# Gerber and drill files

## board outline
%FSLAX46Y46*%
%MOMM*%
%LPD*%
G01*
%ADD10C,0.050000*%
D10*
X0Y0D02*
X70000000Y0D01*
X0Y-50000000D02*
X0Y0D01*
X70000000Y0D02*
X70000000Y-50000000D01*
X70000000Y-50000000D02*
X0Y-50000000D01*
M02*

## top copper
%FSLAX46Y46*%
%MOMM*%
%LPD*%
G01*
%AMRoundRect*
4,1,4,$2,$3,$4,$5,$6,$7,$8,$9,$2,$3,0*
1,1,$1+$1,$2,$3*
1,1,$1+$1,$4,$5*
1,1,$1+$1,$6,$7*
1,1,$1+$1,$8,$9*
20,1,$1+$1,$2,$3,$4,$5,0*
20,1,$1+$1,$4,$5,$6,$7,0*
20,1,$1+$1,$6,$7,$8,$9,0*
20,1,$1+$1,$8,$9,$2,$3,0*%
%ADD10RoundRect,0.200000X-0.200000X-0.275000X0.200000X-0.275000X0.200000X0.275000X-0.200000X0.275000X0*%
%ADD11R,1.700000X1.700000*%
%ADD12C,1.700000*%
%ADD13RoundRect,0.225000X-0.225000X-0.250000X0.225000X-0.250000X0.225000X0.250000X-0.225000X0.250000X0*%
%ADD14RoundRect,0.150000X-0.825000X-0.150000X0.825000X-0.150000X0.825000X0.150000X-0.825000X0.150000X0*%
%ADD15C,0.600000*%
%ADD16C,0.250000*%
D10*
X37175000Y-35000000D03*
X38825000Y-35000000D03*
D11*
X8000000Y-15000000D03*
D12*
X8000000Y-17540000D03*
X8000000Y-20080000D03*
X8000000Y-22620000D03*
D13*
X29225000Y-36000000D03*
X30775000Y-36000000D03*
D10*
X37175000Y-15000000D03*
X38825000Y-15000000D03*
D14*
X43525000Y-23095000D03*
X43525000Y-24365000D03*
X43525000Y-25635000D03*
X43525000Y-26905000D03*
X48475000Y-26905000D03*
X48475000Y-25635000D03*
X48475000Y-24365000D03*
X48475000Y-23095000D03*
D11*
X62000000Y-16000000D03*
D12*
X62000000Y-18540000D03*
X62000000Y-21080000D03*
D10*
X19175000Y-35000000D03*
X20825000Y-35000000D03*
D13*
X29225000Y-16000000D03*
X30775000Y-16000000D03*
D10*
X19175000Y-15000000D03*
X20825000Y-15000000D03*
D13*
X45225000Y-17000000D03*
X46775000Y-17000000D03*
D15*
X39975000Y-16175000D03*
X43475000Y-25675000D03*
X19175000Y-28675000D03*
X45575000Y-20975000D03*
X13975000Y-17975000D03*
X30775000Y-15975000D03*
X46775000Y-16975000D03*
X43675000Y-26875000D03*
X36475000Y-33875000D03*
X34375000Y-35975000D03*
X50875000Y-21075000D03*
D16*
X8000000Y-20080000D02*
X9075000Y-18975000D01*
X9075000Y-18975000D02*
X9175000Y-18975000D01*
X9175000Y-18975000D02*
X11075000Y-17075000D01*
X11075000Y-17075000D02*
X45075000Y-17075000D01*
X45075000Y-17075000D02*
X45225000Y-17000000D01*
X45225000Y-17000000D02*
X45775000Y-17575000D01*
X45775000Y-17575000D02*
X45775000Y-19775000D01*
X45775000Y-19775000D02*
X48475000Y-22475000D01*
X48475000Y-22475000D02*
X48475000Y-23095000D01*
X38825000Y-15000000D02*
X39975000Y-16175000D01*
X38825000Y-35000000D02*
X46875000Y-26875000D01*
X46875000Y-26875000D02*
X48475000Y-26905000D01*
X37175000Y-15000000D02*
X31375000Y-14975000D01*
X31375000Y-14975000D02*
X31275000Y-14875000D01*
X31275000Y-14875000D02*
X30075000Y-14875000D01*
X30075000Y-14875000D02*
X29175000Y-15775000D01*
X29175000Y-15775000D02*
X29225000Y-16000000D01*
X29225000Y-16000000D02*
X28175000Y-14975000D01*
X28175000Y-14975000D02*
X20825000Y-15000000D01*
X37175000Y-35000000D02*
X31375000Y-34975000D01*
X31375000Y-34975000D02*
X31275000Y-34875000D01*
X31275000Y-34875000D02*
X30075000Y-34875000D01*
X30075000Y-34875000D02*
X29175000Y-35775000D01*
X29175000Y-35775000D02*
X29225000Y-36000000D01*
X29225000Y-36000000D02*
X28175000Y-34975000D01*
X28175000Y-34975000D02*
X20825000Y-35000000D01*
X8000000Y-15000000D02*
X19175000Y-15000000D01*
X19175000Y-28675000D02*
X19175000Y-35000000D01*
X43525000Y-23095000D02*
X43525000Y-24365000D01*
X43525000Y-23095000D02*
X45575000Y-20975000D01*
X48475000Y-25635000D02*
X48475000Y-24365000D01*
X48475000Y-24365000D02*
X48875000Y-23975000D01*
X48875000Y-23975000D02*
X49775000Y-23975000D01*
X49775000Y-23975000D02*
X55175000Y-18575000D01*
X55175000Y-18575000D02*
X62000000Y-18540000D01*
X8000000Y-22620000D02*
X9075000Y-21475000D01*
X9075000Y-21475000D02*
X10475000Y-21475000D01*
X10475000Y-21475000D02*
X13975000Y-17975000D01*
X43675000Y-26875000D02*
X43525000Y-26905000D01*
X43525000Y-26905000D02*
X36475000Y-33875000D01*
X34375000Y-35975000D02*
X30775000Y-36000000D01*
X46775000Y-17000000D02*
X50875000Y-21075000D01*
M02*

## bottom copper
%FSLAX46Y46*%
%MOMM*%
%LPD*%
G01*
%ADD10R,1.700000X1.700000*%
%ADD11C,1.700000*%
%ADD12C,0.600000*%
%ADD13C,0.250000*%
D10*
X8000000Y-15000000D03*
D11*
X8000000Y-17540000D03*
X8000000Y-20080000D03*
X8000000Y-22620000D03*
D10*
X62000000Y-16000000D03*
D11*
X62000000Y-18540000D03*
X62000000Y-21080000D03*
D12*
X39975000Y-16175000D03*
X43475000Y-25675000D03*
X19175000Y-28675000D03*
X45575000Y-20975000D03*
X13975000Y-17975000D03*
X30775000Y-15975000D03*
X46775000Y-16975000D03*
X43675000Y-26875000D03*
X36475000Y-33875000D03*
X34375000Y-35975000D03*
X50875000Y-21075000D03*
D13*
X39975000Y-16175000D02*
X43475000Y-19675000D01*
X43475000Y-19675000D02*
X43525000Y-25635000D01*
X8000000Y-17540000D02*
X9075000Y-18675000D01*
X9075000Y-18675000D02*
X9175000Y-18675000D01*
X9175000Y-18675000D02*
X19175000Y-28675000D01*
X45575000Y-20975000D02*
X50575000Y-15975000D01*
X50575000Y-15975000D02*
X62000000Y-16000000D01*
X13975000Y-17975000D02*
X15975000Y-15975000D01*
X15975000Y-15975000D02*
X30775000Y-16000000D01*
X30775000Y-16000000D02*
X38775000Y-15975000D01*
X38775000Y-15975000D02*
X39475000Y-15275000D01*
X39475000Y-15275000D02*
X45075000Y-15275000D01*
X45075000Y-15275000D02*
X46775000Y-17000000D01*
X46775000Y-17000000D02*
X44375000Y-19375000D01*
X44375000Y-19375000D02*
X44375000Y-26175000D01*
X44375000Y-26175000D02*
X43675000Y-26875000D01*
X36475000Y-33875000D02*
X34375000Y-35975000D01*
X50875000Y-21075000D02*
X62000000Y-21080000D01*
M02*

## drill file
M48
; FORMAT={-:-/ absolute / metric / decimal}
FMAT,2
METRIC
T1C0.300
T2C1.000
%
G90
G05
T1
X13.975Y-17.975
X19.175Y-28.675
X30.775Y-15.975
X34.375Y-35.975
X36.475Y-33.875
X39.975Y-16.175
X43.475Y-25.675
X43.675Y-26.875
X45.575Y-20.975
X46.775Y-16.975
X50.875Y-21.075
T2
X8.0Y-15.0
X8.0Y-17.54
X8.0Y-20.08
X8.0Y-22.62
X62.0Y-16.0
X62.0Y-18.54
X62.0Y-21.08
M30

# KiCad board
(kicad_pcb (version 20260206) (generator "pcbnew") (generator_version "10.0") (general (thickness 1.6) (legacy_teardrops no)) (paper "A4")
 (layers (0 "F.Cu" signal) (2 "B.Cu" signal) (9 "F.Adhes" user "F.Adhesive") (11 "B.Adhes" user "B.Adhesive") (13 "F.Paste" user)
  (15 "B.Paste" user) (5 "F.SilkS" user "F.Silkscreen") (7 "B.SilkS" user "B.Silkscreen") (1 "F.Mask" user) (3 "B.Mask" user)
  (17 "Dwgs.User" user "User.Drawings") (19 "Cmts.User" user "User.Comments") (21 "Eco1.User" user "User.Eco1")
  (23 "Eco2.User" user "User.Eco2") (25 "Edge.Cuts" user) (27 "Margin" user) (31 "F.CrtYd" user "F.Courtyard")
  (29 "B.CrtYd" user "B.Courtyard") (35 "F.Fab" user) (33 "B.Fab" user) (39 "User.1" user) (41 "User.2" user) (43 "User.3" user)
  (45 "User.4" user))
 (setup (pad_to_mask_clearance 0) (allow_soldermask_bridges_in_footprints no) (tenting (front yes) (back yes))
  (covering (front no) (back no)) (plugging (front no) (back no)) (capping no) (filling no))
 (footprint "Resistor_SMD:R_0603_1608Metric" (layer "F.Cu") (at 38 35)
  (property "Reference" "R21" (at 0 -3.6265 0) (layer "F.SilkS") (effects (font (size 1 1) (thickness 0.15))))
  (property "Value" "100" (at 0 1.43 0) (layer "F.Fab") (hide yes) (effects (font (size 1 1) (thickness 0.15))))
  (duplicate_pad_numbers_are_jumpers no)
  (pad "1" smd roundrect (at -0.825 0) (size 0.8 0.95) (layers "F.Cu" "F.Mask" "F.Paste") (roundrect_rratio 0.25) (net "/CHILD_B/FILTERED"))
  (pad "2" smd roundrect (at 0.825 0) (size 0.8 0.95) (layers "F.Cu" "F.Mask" "F.Paste") (roundrect_rratio 0.25) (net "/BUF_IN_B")))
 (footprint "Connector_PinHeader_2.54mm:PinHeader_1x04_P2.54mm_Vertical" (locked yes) (layer "F.Cu") (at 8 15)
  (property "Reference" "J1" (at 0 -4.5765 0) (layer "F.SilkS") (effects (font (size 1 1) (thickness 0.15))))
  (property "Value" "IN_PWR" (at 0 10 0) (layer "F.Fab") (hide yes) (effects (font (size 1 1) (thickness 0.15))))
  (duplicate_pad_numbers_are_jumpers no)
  (pad "1" thru_hole rect (at 0 0) (size 1.7 1.7) (drill 1) (layers "*.Cu" "*.Mask") (remove_unused_layers no) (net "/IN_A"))
  (pad "2" thru_hole circle (at 0 2.54) (size 1.7 1.7) (drill 1) (layers "*.Cu" "*.Mask") (remove_unused_layers no) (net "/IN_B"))
  (pad "3" thru_hole circle (at 0 5.08) (size 1.7 1.7) (drill 1) (layers "*.Cu" "*.Mask") (remove_unused_layers no) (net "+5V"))
  (pad "4" thru_hole circle (at 0 7.62) (size 1.7 1.7) (drill 1) (layers "*.Cu" "*.Mask") (remove_unused_layers no) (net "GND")))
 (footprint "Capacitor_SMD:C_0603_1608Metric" (layer "F.Cu") (at 30 36)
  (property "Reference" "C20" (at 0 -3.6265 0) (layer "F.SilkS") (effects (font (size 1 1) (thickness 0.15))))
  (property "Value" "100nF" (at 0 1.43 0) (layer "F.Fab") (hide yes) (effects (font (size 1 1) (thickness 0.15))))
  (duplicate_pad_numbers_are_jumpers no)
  (pad "1" smd roundrect (at -0.775 0) (size 0.9 0.95) (layers "F.Cu" "F.Mask" "F.Paste") (roundrect_rratio 0.25) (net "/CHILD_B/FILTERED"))
  (pad "2" smd roundrect (at 0.775 0) (size 0.9 0.95) (layers "F.Cu" "F.Mask" "F.Paste") (roundrect_rratio 0.25) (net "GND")))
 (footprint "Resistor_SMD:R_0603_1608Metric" (layer "F.Cu") (at 38 15)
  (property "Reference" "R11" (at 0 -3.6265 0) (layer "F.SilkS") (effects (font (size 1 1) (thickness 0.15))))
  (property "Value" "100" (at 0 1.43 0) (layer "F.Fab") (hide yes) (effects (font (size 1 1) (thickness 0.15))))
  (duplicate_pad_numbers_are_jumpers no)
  (pad "1" smd roundrect (at -0.825 0) (size 0.8 0.95) (layers "F.Cu" "F.Mask" "F.Paste") (roundrect_rratio 0.25) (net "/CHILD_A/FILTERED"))
  (pad "2" smd roundrect (at 0.825 0) (size 0.8 0.95) (layers "F.Cu" "F.Mask" "F.Paste") (roundrect_rratio 0.25) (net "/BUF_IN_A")))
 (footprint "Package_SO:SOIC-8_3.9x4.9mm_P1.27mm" (layer "F.Cu") (at 46 25)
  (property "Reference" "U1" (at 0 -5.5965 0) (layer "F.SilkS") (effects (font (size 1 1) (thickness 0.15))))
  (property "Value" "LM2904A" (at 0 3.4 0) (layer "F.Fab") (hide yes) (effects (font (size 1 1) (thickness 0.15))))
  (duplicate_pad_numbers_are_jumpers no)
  (pad "1" smd roundrect (at -2.475 -1.905) (size 1.95 0.6) (layers "F.Cu" "F.Mask" "F.Paste") (roundrect_rratio 0.25) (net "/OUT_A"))
  (pad "2" smd roundrect (at -2.475 -0.635) (size 1.95 0.6) (layers "F.Cu" "F.Mask" "F.Paste") (roundrect_rratio 0.25) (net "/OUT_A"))
  (pad "3" smd roundrect (at -2.475 0.635) (size 1.95 0.6) (layers "F.Cu" "F.Mask" "F.Paste") (roundrect_rratio 0.25) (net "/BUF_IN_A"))
  (pad "4" smd roundrect (at -2.475 1.905) (size 1.95 0.6) (layers "F.Cu" "F.Mask" "F.Paste") (roundrect_rratio 0.25) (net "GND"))
  (pad "5" smd roundrect (at 2.475 1.905) (size 1.95 0.6) (layers "F.Cu" "F.Mask" "F.Paste") (roundrect_rratio 0.25) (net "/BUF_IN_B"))
  (pad "6" smd roundrect (at 2.475 0.635) (size 1.95 0.6) (layers "F.Cu" "F.Mask" "F.Paste") (roundrect_rratio 0.25) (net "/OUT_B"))
  (pad "7" smd roundrect (at 2.475 -0.635) (size 1.95 0.6) (layers "F.Cu" "F.Mask" "F.Paste") (roundrect_rratio 0.25) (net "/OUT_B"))
  (pad "8" smd roundrect (at 2.475 -1.905) (size 1.95 0.6) (layers "F.Cu" "F.Mask" "F.Paste") (roundrect_rratio 0.25) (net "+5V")))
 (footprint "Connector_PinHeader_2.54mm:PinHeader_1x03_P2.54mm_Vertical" (layer "F.Cu") (at 62 16)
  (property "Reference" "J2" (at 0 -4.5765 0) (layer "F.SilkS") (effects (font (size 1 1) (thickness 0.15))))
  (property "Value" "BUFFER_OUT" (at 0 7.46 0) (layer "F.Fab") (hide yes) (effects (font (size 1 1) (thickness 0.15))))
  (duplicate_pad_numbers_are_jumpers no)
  (pad "1" thru_hole rect (at 0 0) (size 1.7 1.7) (drill 1) (layers "*.Cu" "*.Mask") (remove_unused_layers no) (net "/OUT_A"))
  (pad "2" thru_hole circle (at 0 2.54) (size 1.7 1.7) (drill 1) (layers "*.Cu" "*.Mask") (remove_unused_layers no) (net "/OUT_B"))
  (pad "3" thru_hole circle (at 0 5.08) (size 1.7 1.7) (drill 1) (layers "*.Cu" "*.Mask") (remove_unused_layers no) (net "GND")))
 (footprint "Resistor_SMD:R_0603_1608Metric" (layer "F.Cu") (at 20 35)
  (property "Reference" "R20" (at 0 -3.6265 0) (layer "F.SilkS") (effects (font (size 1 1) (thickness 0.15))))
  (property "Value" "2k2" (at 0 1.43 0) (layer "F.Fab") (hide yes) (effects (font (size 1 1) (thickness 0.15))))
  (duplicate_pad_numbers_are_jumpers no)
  (pad "1" smd roundrect (at -0.825 0) (size 0.8 0.95) (layers "F.Cu" "F.Mask" "F.Paste") (roundrect_rratio 0.25) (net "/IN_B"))
  (pad "2" smd roundrect (at 0.825 0) (size 0.8 0.95) (layers "F.Cu" "F.Mask" "F.Paste") (roundrect_rratio 0.25) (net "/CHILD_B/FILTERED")))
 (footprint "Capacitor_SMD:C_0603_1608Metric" (layer "F.Cu") (at 30 16)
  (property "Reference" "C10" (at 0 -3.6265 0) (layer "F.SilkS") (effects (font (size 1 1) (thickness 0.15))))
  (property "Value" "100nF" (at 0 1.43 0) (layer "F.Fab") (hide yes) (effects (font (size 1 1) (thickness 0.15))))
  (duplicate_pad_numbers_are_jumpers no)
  (pad "1" smd roundrect (at -0.775 0) (size 0.9 0.95) (layers "F.Cu" "F.Mask" "F.Paste") (roundrect_rratio 0.25) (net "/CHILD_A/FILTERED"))
  (pad "2" smd roundrect (at 0.775 0) (size 0.9 0.95) (layers "F.Cu" "F.Mask" "F.Paste") (roundrect_rratio 0.25) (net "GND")))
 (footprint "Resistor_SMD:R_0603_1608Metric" (layer "F.Cu") (at 20 15)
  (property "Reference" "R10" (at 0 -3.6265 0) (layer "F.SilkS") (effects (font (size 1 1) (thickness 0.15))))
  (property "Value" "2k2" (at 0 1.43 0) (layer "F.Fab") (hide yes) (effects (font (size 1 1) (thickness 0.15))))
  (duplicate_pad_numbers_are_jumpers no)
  (pad "1" smd roundrect (at -0.825 0) (size 0.8 0.95) (layers "F.Cu" "F.Mask" "F.Paste") (roundrect_rratio 0.25) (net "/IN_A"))
  (pad "2" smd roundrect (at 0.825 0) (size 0.8 0.95) (layers "F.Cu" "F.Mask" "F.Paste") (roundrect_rratio 0.25) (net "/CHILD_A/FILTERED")))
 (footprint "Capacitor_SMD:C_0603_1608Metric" (layer "F.Cu") (at 46 17)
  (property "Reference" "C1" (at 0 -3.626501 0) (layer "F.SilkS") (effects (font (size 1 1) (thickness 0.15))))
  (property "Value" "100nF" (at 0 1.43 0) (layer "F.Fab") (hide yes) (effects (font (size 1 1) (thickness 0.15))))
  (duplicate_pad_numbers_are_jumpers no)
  (pad "1" smd roundrect (at -0.775 0) (size 0.9 0.95) (layers "F.Cu" "F.Mask" "F.Paste") (roundrect_rratio 0.25) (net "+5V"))
  (pad "2" smd roundrect (at 0.775 0) (size 0.9 0.95) (layers "F.Cu" "F.Mask" "F.Paste") (roundrect_rratio 0.25) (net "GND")))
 (gr_line (start 0 0) (end 70 0) (stroke (width 0.05) (type default)) (layer "Edge.Cuts"))
 (gr_line (start 0 50) (end 0 0) (stroke (width 0.05) (type default)) (layer "Edge.Cuts"))
 (gr_line (start 70 0) (end 70 50) (stroke (width 0.05) (type default)) (layer "Edge.Cuts"))
 (gr_line (start 70 50) (end 0 50) (stroke (width 0.05) (type default)) (layer "Edge.Cuts"))
 (segment (start 8 20.08) (end 9.075 18.975) (width 0.25) (layer "F.Cu") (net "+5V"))
 (segment (start 9.075 18.975) (end 9.175 18.975) (width 0.25) (layer "F.Cu") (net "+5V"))
 (segment (start 9.175 18.975) (end 11.075 17.075) (width 0.25) (layer "F.Cu") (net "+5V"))
 (segment (start 11.075 17.075) (end 45.075 17.075) (width 0.25) (layer "F.Cu") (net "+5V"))
 (segment (start 45.075 17.075) (end 45.225 17) (width 0.25) (layer "F.Cu") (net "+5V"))
 (segment (start 45.225 17) (end 45.775 17.575) (width 0.25) (layer "F.Cu") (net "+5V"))
 (segment (start 45.775 17.575) (end 45.775 19.775) (width 0.25) (layer "F.Cu") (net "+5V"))
 (segment (start 45.775 19.775) (end 48.475 22.475) (width 0.25) (layer "F.Cu") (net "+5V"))
 (segment (start 48.475 22.475) (end 48.475 23.095) (width 0.25) (layer "F.Cu") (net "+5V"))
 (segment (start 38.825 15) (end 39.975 16.175) (width 0.25) (layer "F.Cu") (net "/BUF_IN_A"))
 (via (at 39.975 16.175) (size 0.6) (drill 0.3) (layers "F.Cu" "B.Cu") (capping no) (covering (front no) (back no))
  (plugging (front no) (back no)) (filling no) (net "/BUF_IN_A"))
 (segment (start 39.975 16.175) (end 43.475 19.675) (width 0.25) (layer "B.Cu") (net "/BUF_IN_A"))
 (segment (start 43.475 19.675) (end 43.525 25.635) (width 0.25) (layer "B.Cu") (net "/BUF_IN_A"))
 (via (at 43.475 25.675) (size 0.6) (drill 0.3) (layers "F.Cu" "B.Cu") (capping no) (covering (front no) (back no))
  (plugging (front no) (back no)) (filling no) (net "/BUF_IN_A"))
 (segment (start 38.825 35) (end 46.875 26.875) (width 0.25) (layer "F.Cu") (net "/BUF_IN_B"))
 (segment (start 46.875 26.875) (end 48.475 26.905) (width 0.25) (layer "F.Cu") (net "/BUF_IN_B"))
 (segment (start 37.175 15) (end 31.375 14.975) (width 0.25) (layer "F.Cu") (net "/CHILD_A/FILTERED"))
 (segment (start 31.375 14.975) (end 31.275 14.875) (width 0.25) (layer "F.Cu") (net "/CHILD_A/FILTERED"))
 (segment (start 31.275 14.875) (end 30.075 14.875) (width 0.25) (layer "F.Cu") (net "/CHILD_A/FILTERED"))
 (segment (start 30.075 14.875) (end 29.175 15.775) (width 0.25) (layer "F.Cu") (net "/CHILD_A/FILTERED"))
 (segment (start 29.175 15.775) (end 29.225 16) (width 0.25) (layer "F.Cu") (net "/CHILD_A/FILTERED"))
 (segment (start 29.225 16) (end 28.175 14.975) (width 0.25) (layer "F.Cu") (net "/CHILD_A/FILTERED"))
 (segment (start 28.175 14.975) (end 20.825 15) (width 0.25) (layer "F.Cu") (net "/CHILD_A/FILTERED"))
 (segment (start 37.175 35) (end 31.375 34.975) (width 0.25) (layer "F.Cu") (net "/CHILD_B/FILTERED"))
 (segment (start 31.375 34.975) (end 31.275 34.875) (width 0.25) (layer "F.Cu") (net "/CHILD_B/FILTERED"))
 (segment (start 31.275 34.875) (end 30.075 34.875) (width 0.25) (layer "F.Cu") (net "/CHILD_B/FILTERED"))
 (segment (start 30.075 34.875) (end 29.175 35.775) (width 0.25) (layer "F.Cu") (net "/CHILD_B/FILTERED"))
 (segment (start 29.175 35.775) (end 29.225 36) (width 0.25) (layer "F.Cu") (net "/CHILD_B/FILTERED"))
 (segment (start 29.225 36) (end 28.175 34.975) (width 0.25) (layer "F.Cu") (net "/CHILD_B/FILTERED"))
 (segment (start 28.175 34.975) (end 20.825 35) (width 0.25) (layer "F.Cu") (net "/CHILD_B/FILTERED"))
 (segment (start 8 15) (end 19.175 15) (width 0.25) (layer "F.Cu") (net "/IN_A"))
 (segment (start 8 17.54) (end 9.075 18.675) (width 0.25) (layer "B.Cu") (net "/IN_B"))
 (segment (start 9.075 18.675) (end 9.175 18.675) (width 0.25) (layer "B.Cu") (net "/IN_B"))
 (segment (start 9.175 18.675) (end 19.175 28.675) (width 0.25) (layer "B.Cu") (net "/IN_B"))
 (via (at 19.175 28.675) (size 0.6) (drill 0.3) (layers "F.Cu" "B.Cu") (capping no) (covering (front no) (back no))
  (plugging (front no) (back no)) (filling no) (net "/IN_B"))
 (segment (start 19.175 28.675) (end 19.175 35) (width 0.25) (layer "F.Cu") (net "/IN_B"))
 (segment (start 43.525 23.095) (end 43.525 24.365) (width 0.25) (layer "F.Cu") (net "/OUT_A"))
 (segment (start 43.525 23.095) (end 45.575 20.975) (width 0.25) (layer "F.Cu") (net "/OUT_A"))
 (via (at 45.575 20.975) (size 0.6) (drill 0.3) (layers "F.Cu" "B.Cu") (capping no) (covering (front no) (back no))
  (plugging (front no) (back no)) (filling no) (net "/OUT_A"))
 (segment (start 45.575 20.975) (end 50.575 15.975) (width 0.25) (layer "B.Cu") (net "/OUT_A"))
 (segment (start 50.575 15.975) (end 62 16) (width 0.25) (layer "B.Cu") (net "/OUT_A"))
 (segment (start 48.475 25.635) (end 48.475 24.365) (width 0.25) (layer "F.Cu") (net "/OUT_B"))
 (segment (start 48.475 24.365) (end 48.875 23.975) (width 0.25) (layer "F.Cu") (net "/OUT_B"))
 (segment (start 48.875 23.975) (end 49.775 23.975) (width 0.25) (layer "F.Cu") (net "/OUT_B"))
 (segment (start 49.775 23.975) (end 55.175 18.575) (width 0.25) (layer "F.Cu") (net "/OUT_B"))
 (segment (start 55.175 18.575) (end 62 18.54) (width 0.25) (layer "F.Cu") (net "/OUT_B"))
 (segment (start 8 22.62) (end 9.075 21.475) (width 0.25) (layer "F.Cu") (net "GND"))
 (segment (start 9.075 21.475) (end 10.475 21.475) (width 0.25) (layer "F.Cu") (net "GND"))
 (segment (start 10.475 21.475) (end 13.975 17.975) (width 0.25) (layer "F.Cu") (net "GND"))
 (via (at 13.975 17.975) (size 0.6) (drill 0.3) (layers "F.Cu" "B.Cu") (capping no) (covering (front no) (back no))
  (plugging (front no) (back no)) (filling no) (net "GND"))
 (segment (start 13.975 17.975) (end 15.975 15.975) (width 0.25) (layer "B.Cu") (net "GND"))
 (segment (start 15.975 15.975) (end 30.775 16) (width 0.25) (layer "B.Cu") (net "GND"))
 (via (at 30.775 15.975) (size 0.6) (drill 0.3) (layers "F.Cu" "B.Cu") (capping no) (covering (front no) (back no))
  (plugging (front no) (back no)) (filling no) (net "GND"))
 (segment (start 30.775 16) (end 38.775 15.975) (width 0.25) (layer "B.Cu") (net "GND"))
 (segment (start 38.775 15.975) (end 39.475 15.275) (width 0.25) (layer "B.Cu") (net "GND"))
 (segment (start 39.475 15.275) (end 45.075 15.275) (width 0.25) (layer "B.Cu") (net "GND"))
 (segment (start 45.075 15.275) (end 46.775 17) (width 0.25) (layer "B.Cu") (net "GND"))
 (via (at 46.775 16.975) (size 0.6) (drill 0.3) (layers "F.Cu" "B.Cu") (capping no) (covering (front no) (back no))
  (plugging (front no) (back no)) (filling no) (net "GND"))
 (segment (start 46.775 17) (end 44.375 19.375) (width 0.25) (layer "B.Cu") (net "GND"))
 (segment (start 44.375 19.375) (end 44.375 26.175) (width 0.25) (layer "B.Cu") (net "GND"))
 (segment (start 44.375 26.175) (end 43.675 26.875) (width 0.25) (layer "B.Cu") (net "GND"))
 (via (at 43.675 26.875) (size 0.6) (drill 0.3) (layers "F.Cu" "B.Cu") (capping no) (covering (front no) (back no))
  (plugging (front no) (back no)) (filling no) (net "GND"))
 (segment (start 43.675 26.875) (end 43.525 26.905) (width 0.25) (layer "F.Cu") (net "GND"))
 (segment (start 43.525 26.905) (end 36.475 33.875) (width 0.25) (layer "F.Cu") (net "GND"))
 (via (at 36.475 33.875) (size 0.6) (drill 0.3) (layers "F.Cu" "B.Cu") (capping no) (covering (front no) (back no))
  (plugging (front no) (back no)) (filling no) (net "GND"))
 (segment (start 36.475 33.875) (end 34.375 35.975) (width 0.25) (layer "B.Cu") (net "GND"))
 (via (at 34.375 35.975) (size 0.6) (drill 0.3) (layers "F.Cu" "B.Cu") (capping no) (covering (front no) (back no))
  (plugging (front no) (back no)) (filling no) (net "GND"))
 (segment (start 34.375 35.975) (end 30.775 36) (width 0.25) (layer "F.Cu") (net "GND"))
 (segment (start 46.775 17) (end 50.875 21.075) (width 0.25) (layer "F.Cu") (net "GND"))
 (via (at 50.875 21.075) (size 0.6) (drill 0.3) (layers "F.Cu" "B.Cu") (capping no) (covering (front no) (back no))
  (plugging (front no) (back no)) (filling no) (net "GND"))
 (segment (start 50.875 21.075) (end 62 21.08) (width 0.25) (layer "B.Cu") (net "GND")))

